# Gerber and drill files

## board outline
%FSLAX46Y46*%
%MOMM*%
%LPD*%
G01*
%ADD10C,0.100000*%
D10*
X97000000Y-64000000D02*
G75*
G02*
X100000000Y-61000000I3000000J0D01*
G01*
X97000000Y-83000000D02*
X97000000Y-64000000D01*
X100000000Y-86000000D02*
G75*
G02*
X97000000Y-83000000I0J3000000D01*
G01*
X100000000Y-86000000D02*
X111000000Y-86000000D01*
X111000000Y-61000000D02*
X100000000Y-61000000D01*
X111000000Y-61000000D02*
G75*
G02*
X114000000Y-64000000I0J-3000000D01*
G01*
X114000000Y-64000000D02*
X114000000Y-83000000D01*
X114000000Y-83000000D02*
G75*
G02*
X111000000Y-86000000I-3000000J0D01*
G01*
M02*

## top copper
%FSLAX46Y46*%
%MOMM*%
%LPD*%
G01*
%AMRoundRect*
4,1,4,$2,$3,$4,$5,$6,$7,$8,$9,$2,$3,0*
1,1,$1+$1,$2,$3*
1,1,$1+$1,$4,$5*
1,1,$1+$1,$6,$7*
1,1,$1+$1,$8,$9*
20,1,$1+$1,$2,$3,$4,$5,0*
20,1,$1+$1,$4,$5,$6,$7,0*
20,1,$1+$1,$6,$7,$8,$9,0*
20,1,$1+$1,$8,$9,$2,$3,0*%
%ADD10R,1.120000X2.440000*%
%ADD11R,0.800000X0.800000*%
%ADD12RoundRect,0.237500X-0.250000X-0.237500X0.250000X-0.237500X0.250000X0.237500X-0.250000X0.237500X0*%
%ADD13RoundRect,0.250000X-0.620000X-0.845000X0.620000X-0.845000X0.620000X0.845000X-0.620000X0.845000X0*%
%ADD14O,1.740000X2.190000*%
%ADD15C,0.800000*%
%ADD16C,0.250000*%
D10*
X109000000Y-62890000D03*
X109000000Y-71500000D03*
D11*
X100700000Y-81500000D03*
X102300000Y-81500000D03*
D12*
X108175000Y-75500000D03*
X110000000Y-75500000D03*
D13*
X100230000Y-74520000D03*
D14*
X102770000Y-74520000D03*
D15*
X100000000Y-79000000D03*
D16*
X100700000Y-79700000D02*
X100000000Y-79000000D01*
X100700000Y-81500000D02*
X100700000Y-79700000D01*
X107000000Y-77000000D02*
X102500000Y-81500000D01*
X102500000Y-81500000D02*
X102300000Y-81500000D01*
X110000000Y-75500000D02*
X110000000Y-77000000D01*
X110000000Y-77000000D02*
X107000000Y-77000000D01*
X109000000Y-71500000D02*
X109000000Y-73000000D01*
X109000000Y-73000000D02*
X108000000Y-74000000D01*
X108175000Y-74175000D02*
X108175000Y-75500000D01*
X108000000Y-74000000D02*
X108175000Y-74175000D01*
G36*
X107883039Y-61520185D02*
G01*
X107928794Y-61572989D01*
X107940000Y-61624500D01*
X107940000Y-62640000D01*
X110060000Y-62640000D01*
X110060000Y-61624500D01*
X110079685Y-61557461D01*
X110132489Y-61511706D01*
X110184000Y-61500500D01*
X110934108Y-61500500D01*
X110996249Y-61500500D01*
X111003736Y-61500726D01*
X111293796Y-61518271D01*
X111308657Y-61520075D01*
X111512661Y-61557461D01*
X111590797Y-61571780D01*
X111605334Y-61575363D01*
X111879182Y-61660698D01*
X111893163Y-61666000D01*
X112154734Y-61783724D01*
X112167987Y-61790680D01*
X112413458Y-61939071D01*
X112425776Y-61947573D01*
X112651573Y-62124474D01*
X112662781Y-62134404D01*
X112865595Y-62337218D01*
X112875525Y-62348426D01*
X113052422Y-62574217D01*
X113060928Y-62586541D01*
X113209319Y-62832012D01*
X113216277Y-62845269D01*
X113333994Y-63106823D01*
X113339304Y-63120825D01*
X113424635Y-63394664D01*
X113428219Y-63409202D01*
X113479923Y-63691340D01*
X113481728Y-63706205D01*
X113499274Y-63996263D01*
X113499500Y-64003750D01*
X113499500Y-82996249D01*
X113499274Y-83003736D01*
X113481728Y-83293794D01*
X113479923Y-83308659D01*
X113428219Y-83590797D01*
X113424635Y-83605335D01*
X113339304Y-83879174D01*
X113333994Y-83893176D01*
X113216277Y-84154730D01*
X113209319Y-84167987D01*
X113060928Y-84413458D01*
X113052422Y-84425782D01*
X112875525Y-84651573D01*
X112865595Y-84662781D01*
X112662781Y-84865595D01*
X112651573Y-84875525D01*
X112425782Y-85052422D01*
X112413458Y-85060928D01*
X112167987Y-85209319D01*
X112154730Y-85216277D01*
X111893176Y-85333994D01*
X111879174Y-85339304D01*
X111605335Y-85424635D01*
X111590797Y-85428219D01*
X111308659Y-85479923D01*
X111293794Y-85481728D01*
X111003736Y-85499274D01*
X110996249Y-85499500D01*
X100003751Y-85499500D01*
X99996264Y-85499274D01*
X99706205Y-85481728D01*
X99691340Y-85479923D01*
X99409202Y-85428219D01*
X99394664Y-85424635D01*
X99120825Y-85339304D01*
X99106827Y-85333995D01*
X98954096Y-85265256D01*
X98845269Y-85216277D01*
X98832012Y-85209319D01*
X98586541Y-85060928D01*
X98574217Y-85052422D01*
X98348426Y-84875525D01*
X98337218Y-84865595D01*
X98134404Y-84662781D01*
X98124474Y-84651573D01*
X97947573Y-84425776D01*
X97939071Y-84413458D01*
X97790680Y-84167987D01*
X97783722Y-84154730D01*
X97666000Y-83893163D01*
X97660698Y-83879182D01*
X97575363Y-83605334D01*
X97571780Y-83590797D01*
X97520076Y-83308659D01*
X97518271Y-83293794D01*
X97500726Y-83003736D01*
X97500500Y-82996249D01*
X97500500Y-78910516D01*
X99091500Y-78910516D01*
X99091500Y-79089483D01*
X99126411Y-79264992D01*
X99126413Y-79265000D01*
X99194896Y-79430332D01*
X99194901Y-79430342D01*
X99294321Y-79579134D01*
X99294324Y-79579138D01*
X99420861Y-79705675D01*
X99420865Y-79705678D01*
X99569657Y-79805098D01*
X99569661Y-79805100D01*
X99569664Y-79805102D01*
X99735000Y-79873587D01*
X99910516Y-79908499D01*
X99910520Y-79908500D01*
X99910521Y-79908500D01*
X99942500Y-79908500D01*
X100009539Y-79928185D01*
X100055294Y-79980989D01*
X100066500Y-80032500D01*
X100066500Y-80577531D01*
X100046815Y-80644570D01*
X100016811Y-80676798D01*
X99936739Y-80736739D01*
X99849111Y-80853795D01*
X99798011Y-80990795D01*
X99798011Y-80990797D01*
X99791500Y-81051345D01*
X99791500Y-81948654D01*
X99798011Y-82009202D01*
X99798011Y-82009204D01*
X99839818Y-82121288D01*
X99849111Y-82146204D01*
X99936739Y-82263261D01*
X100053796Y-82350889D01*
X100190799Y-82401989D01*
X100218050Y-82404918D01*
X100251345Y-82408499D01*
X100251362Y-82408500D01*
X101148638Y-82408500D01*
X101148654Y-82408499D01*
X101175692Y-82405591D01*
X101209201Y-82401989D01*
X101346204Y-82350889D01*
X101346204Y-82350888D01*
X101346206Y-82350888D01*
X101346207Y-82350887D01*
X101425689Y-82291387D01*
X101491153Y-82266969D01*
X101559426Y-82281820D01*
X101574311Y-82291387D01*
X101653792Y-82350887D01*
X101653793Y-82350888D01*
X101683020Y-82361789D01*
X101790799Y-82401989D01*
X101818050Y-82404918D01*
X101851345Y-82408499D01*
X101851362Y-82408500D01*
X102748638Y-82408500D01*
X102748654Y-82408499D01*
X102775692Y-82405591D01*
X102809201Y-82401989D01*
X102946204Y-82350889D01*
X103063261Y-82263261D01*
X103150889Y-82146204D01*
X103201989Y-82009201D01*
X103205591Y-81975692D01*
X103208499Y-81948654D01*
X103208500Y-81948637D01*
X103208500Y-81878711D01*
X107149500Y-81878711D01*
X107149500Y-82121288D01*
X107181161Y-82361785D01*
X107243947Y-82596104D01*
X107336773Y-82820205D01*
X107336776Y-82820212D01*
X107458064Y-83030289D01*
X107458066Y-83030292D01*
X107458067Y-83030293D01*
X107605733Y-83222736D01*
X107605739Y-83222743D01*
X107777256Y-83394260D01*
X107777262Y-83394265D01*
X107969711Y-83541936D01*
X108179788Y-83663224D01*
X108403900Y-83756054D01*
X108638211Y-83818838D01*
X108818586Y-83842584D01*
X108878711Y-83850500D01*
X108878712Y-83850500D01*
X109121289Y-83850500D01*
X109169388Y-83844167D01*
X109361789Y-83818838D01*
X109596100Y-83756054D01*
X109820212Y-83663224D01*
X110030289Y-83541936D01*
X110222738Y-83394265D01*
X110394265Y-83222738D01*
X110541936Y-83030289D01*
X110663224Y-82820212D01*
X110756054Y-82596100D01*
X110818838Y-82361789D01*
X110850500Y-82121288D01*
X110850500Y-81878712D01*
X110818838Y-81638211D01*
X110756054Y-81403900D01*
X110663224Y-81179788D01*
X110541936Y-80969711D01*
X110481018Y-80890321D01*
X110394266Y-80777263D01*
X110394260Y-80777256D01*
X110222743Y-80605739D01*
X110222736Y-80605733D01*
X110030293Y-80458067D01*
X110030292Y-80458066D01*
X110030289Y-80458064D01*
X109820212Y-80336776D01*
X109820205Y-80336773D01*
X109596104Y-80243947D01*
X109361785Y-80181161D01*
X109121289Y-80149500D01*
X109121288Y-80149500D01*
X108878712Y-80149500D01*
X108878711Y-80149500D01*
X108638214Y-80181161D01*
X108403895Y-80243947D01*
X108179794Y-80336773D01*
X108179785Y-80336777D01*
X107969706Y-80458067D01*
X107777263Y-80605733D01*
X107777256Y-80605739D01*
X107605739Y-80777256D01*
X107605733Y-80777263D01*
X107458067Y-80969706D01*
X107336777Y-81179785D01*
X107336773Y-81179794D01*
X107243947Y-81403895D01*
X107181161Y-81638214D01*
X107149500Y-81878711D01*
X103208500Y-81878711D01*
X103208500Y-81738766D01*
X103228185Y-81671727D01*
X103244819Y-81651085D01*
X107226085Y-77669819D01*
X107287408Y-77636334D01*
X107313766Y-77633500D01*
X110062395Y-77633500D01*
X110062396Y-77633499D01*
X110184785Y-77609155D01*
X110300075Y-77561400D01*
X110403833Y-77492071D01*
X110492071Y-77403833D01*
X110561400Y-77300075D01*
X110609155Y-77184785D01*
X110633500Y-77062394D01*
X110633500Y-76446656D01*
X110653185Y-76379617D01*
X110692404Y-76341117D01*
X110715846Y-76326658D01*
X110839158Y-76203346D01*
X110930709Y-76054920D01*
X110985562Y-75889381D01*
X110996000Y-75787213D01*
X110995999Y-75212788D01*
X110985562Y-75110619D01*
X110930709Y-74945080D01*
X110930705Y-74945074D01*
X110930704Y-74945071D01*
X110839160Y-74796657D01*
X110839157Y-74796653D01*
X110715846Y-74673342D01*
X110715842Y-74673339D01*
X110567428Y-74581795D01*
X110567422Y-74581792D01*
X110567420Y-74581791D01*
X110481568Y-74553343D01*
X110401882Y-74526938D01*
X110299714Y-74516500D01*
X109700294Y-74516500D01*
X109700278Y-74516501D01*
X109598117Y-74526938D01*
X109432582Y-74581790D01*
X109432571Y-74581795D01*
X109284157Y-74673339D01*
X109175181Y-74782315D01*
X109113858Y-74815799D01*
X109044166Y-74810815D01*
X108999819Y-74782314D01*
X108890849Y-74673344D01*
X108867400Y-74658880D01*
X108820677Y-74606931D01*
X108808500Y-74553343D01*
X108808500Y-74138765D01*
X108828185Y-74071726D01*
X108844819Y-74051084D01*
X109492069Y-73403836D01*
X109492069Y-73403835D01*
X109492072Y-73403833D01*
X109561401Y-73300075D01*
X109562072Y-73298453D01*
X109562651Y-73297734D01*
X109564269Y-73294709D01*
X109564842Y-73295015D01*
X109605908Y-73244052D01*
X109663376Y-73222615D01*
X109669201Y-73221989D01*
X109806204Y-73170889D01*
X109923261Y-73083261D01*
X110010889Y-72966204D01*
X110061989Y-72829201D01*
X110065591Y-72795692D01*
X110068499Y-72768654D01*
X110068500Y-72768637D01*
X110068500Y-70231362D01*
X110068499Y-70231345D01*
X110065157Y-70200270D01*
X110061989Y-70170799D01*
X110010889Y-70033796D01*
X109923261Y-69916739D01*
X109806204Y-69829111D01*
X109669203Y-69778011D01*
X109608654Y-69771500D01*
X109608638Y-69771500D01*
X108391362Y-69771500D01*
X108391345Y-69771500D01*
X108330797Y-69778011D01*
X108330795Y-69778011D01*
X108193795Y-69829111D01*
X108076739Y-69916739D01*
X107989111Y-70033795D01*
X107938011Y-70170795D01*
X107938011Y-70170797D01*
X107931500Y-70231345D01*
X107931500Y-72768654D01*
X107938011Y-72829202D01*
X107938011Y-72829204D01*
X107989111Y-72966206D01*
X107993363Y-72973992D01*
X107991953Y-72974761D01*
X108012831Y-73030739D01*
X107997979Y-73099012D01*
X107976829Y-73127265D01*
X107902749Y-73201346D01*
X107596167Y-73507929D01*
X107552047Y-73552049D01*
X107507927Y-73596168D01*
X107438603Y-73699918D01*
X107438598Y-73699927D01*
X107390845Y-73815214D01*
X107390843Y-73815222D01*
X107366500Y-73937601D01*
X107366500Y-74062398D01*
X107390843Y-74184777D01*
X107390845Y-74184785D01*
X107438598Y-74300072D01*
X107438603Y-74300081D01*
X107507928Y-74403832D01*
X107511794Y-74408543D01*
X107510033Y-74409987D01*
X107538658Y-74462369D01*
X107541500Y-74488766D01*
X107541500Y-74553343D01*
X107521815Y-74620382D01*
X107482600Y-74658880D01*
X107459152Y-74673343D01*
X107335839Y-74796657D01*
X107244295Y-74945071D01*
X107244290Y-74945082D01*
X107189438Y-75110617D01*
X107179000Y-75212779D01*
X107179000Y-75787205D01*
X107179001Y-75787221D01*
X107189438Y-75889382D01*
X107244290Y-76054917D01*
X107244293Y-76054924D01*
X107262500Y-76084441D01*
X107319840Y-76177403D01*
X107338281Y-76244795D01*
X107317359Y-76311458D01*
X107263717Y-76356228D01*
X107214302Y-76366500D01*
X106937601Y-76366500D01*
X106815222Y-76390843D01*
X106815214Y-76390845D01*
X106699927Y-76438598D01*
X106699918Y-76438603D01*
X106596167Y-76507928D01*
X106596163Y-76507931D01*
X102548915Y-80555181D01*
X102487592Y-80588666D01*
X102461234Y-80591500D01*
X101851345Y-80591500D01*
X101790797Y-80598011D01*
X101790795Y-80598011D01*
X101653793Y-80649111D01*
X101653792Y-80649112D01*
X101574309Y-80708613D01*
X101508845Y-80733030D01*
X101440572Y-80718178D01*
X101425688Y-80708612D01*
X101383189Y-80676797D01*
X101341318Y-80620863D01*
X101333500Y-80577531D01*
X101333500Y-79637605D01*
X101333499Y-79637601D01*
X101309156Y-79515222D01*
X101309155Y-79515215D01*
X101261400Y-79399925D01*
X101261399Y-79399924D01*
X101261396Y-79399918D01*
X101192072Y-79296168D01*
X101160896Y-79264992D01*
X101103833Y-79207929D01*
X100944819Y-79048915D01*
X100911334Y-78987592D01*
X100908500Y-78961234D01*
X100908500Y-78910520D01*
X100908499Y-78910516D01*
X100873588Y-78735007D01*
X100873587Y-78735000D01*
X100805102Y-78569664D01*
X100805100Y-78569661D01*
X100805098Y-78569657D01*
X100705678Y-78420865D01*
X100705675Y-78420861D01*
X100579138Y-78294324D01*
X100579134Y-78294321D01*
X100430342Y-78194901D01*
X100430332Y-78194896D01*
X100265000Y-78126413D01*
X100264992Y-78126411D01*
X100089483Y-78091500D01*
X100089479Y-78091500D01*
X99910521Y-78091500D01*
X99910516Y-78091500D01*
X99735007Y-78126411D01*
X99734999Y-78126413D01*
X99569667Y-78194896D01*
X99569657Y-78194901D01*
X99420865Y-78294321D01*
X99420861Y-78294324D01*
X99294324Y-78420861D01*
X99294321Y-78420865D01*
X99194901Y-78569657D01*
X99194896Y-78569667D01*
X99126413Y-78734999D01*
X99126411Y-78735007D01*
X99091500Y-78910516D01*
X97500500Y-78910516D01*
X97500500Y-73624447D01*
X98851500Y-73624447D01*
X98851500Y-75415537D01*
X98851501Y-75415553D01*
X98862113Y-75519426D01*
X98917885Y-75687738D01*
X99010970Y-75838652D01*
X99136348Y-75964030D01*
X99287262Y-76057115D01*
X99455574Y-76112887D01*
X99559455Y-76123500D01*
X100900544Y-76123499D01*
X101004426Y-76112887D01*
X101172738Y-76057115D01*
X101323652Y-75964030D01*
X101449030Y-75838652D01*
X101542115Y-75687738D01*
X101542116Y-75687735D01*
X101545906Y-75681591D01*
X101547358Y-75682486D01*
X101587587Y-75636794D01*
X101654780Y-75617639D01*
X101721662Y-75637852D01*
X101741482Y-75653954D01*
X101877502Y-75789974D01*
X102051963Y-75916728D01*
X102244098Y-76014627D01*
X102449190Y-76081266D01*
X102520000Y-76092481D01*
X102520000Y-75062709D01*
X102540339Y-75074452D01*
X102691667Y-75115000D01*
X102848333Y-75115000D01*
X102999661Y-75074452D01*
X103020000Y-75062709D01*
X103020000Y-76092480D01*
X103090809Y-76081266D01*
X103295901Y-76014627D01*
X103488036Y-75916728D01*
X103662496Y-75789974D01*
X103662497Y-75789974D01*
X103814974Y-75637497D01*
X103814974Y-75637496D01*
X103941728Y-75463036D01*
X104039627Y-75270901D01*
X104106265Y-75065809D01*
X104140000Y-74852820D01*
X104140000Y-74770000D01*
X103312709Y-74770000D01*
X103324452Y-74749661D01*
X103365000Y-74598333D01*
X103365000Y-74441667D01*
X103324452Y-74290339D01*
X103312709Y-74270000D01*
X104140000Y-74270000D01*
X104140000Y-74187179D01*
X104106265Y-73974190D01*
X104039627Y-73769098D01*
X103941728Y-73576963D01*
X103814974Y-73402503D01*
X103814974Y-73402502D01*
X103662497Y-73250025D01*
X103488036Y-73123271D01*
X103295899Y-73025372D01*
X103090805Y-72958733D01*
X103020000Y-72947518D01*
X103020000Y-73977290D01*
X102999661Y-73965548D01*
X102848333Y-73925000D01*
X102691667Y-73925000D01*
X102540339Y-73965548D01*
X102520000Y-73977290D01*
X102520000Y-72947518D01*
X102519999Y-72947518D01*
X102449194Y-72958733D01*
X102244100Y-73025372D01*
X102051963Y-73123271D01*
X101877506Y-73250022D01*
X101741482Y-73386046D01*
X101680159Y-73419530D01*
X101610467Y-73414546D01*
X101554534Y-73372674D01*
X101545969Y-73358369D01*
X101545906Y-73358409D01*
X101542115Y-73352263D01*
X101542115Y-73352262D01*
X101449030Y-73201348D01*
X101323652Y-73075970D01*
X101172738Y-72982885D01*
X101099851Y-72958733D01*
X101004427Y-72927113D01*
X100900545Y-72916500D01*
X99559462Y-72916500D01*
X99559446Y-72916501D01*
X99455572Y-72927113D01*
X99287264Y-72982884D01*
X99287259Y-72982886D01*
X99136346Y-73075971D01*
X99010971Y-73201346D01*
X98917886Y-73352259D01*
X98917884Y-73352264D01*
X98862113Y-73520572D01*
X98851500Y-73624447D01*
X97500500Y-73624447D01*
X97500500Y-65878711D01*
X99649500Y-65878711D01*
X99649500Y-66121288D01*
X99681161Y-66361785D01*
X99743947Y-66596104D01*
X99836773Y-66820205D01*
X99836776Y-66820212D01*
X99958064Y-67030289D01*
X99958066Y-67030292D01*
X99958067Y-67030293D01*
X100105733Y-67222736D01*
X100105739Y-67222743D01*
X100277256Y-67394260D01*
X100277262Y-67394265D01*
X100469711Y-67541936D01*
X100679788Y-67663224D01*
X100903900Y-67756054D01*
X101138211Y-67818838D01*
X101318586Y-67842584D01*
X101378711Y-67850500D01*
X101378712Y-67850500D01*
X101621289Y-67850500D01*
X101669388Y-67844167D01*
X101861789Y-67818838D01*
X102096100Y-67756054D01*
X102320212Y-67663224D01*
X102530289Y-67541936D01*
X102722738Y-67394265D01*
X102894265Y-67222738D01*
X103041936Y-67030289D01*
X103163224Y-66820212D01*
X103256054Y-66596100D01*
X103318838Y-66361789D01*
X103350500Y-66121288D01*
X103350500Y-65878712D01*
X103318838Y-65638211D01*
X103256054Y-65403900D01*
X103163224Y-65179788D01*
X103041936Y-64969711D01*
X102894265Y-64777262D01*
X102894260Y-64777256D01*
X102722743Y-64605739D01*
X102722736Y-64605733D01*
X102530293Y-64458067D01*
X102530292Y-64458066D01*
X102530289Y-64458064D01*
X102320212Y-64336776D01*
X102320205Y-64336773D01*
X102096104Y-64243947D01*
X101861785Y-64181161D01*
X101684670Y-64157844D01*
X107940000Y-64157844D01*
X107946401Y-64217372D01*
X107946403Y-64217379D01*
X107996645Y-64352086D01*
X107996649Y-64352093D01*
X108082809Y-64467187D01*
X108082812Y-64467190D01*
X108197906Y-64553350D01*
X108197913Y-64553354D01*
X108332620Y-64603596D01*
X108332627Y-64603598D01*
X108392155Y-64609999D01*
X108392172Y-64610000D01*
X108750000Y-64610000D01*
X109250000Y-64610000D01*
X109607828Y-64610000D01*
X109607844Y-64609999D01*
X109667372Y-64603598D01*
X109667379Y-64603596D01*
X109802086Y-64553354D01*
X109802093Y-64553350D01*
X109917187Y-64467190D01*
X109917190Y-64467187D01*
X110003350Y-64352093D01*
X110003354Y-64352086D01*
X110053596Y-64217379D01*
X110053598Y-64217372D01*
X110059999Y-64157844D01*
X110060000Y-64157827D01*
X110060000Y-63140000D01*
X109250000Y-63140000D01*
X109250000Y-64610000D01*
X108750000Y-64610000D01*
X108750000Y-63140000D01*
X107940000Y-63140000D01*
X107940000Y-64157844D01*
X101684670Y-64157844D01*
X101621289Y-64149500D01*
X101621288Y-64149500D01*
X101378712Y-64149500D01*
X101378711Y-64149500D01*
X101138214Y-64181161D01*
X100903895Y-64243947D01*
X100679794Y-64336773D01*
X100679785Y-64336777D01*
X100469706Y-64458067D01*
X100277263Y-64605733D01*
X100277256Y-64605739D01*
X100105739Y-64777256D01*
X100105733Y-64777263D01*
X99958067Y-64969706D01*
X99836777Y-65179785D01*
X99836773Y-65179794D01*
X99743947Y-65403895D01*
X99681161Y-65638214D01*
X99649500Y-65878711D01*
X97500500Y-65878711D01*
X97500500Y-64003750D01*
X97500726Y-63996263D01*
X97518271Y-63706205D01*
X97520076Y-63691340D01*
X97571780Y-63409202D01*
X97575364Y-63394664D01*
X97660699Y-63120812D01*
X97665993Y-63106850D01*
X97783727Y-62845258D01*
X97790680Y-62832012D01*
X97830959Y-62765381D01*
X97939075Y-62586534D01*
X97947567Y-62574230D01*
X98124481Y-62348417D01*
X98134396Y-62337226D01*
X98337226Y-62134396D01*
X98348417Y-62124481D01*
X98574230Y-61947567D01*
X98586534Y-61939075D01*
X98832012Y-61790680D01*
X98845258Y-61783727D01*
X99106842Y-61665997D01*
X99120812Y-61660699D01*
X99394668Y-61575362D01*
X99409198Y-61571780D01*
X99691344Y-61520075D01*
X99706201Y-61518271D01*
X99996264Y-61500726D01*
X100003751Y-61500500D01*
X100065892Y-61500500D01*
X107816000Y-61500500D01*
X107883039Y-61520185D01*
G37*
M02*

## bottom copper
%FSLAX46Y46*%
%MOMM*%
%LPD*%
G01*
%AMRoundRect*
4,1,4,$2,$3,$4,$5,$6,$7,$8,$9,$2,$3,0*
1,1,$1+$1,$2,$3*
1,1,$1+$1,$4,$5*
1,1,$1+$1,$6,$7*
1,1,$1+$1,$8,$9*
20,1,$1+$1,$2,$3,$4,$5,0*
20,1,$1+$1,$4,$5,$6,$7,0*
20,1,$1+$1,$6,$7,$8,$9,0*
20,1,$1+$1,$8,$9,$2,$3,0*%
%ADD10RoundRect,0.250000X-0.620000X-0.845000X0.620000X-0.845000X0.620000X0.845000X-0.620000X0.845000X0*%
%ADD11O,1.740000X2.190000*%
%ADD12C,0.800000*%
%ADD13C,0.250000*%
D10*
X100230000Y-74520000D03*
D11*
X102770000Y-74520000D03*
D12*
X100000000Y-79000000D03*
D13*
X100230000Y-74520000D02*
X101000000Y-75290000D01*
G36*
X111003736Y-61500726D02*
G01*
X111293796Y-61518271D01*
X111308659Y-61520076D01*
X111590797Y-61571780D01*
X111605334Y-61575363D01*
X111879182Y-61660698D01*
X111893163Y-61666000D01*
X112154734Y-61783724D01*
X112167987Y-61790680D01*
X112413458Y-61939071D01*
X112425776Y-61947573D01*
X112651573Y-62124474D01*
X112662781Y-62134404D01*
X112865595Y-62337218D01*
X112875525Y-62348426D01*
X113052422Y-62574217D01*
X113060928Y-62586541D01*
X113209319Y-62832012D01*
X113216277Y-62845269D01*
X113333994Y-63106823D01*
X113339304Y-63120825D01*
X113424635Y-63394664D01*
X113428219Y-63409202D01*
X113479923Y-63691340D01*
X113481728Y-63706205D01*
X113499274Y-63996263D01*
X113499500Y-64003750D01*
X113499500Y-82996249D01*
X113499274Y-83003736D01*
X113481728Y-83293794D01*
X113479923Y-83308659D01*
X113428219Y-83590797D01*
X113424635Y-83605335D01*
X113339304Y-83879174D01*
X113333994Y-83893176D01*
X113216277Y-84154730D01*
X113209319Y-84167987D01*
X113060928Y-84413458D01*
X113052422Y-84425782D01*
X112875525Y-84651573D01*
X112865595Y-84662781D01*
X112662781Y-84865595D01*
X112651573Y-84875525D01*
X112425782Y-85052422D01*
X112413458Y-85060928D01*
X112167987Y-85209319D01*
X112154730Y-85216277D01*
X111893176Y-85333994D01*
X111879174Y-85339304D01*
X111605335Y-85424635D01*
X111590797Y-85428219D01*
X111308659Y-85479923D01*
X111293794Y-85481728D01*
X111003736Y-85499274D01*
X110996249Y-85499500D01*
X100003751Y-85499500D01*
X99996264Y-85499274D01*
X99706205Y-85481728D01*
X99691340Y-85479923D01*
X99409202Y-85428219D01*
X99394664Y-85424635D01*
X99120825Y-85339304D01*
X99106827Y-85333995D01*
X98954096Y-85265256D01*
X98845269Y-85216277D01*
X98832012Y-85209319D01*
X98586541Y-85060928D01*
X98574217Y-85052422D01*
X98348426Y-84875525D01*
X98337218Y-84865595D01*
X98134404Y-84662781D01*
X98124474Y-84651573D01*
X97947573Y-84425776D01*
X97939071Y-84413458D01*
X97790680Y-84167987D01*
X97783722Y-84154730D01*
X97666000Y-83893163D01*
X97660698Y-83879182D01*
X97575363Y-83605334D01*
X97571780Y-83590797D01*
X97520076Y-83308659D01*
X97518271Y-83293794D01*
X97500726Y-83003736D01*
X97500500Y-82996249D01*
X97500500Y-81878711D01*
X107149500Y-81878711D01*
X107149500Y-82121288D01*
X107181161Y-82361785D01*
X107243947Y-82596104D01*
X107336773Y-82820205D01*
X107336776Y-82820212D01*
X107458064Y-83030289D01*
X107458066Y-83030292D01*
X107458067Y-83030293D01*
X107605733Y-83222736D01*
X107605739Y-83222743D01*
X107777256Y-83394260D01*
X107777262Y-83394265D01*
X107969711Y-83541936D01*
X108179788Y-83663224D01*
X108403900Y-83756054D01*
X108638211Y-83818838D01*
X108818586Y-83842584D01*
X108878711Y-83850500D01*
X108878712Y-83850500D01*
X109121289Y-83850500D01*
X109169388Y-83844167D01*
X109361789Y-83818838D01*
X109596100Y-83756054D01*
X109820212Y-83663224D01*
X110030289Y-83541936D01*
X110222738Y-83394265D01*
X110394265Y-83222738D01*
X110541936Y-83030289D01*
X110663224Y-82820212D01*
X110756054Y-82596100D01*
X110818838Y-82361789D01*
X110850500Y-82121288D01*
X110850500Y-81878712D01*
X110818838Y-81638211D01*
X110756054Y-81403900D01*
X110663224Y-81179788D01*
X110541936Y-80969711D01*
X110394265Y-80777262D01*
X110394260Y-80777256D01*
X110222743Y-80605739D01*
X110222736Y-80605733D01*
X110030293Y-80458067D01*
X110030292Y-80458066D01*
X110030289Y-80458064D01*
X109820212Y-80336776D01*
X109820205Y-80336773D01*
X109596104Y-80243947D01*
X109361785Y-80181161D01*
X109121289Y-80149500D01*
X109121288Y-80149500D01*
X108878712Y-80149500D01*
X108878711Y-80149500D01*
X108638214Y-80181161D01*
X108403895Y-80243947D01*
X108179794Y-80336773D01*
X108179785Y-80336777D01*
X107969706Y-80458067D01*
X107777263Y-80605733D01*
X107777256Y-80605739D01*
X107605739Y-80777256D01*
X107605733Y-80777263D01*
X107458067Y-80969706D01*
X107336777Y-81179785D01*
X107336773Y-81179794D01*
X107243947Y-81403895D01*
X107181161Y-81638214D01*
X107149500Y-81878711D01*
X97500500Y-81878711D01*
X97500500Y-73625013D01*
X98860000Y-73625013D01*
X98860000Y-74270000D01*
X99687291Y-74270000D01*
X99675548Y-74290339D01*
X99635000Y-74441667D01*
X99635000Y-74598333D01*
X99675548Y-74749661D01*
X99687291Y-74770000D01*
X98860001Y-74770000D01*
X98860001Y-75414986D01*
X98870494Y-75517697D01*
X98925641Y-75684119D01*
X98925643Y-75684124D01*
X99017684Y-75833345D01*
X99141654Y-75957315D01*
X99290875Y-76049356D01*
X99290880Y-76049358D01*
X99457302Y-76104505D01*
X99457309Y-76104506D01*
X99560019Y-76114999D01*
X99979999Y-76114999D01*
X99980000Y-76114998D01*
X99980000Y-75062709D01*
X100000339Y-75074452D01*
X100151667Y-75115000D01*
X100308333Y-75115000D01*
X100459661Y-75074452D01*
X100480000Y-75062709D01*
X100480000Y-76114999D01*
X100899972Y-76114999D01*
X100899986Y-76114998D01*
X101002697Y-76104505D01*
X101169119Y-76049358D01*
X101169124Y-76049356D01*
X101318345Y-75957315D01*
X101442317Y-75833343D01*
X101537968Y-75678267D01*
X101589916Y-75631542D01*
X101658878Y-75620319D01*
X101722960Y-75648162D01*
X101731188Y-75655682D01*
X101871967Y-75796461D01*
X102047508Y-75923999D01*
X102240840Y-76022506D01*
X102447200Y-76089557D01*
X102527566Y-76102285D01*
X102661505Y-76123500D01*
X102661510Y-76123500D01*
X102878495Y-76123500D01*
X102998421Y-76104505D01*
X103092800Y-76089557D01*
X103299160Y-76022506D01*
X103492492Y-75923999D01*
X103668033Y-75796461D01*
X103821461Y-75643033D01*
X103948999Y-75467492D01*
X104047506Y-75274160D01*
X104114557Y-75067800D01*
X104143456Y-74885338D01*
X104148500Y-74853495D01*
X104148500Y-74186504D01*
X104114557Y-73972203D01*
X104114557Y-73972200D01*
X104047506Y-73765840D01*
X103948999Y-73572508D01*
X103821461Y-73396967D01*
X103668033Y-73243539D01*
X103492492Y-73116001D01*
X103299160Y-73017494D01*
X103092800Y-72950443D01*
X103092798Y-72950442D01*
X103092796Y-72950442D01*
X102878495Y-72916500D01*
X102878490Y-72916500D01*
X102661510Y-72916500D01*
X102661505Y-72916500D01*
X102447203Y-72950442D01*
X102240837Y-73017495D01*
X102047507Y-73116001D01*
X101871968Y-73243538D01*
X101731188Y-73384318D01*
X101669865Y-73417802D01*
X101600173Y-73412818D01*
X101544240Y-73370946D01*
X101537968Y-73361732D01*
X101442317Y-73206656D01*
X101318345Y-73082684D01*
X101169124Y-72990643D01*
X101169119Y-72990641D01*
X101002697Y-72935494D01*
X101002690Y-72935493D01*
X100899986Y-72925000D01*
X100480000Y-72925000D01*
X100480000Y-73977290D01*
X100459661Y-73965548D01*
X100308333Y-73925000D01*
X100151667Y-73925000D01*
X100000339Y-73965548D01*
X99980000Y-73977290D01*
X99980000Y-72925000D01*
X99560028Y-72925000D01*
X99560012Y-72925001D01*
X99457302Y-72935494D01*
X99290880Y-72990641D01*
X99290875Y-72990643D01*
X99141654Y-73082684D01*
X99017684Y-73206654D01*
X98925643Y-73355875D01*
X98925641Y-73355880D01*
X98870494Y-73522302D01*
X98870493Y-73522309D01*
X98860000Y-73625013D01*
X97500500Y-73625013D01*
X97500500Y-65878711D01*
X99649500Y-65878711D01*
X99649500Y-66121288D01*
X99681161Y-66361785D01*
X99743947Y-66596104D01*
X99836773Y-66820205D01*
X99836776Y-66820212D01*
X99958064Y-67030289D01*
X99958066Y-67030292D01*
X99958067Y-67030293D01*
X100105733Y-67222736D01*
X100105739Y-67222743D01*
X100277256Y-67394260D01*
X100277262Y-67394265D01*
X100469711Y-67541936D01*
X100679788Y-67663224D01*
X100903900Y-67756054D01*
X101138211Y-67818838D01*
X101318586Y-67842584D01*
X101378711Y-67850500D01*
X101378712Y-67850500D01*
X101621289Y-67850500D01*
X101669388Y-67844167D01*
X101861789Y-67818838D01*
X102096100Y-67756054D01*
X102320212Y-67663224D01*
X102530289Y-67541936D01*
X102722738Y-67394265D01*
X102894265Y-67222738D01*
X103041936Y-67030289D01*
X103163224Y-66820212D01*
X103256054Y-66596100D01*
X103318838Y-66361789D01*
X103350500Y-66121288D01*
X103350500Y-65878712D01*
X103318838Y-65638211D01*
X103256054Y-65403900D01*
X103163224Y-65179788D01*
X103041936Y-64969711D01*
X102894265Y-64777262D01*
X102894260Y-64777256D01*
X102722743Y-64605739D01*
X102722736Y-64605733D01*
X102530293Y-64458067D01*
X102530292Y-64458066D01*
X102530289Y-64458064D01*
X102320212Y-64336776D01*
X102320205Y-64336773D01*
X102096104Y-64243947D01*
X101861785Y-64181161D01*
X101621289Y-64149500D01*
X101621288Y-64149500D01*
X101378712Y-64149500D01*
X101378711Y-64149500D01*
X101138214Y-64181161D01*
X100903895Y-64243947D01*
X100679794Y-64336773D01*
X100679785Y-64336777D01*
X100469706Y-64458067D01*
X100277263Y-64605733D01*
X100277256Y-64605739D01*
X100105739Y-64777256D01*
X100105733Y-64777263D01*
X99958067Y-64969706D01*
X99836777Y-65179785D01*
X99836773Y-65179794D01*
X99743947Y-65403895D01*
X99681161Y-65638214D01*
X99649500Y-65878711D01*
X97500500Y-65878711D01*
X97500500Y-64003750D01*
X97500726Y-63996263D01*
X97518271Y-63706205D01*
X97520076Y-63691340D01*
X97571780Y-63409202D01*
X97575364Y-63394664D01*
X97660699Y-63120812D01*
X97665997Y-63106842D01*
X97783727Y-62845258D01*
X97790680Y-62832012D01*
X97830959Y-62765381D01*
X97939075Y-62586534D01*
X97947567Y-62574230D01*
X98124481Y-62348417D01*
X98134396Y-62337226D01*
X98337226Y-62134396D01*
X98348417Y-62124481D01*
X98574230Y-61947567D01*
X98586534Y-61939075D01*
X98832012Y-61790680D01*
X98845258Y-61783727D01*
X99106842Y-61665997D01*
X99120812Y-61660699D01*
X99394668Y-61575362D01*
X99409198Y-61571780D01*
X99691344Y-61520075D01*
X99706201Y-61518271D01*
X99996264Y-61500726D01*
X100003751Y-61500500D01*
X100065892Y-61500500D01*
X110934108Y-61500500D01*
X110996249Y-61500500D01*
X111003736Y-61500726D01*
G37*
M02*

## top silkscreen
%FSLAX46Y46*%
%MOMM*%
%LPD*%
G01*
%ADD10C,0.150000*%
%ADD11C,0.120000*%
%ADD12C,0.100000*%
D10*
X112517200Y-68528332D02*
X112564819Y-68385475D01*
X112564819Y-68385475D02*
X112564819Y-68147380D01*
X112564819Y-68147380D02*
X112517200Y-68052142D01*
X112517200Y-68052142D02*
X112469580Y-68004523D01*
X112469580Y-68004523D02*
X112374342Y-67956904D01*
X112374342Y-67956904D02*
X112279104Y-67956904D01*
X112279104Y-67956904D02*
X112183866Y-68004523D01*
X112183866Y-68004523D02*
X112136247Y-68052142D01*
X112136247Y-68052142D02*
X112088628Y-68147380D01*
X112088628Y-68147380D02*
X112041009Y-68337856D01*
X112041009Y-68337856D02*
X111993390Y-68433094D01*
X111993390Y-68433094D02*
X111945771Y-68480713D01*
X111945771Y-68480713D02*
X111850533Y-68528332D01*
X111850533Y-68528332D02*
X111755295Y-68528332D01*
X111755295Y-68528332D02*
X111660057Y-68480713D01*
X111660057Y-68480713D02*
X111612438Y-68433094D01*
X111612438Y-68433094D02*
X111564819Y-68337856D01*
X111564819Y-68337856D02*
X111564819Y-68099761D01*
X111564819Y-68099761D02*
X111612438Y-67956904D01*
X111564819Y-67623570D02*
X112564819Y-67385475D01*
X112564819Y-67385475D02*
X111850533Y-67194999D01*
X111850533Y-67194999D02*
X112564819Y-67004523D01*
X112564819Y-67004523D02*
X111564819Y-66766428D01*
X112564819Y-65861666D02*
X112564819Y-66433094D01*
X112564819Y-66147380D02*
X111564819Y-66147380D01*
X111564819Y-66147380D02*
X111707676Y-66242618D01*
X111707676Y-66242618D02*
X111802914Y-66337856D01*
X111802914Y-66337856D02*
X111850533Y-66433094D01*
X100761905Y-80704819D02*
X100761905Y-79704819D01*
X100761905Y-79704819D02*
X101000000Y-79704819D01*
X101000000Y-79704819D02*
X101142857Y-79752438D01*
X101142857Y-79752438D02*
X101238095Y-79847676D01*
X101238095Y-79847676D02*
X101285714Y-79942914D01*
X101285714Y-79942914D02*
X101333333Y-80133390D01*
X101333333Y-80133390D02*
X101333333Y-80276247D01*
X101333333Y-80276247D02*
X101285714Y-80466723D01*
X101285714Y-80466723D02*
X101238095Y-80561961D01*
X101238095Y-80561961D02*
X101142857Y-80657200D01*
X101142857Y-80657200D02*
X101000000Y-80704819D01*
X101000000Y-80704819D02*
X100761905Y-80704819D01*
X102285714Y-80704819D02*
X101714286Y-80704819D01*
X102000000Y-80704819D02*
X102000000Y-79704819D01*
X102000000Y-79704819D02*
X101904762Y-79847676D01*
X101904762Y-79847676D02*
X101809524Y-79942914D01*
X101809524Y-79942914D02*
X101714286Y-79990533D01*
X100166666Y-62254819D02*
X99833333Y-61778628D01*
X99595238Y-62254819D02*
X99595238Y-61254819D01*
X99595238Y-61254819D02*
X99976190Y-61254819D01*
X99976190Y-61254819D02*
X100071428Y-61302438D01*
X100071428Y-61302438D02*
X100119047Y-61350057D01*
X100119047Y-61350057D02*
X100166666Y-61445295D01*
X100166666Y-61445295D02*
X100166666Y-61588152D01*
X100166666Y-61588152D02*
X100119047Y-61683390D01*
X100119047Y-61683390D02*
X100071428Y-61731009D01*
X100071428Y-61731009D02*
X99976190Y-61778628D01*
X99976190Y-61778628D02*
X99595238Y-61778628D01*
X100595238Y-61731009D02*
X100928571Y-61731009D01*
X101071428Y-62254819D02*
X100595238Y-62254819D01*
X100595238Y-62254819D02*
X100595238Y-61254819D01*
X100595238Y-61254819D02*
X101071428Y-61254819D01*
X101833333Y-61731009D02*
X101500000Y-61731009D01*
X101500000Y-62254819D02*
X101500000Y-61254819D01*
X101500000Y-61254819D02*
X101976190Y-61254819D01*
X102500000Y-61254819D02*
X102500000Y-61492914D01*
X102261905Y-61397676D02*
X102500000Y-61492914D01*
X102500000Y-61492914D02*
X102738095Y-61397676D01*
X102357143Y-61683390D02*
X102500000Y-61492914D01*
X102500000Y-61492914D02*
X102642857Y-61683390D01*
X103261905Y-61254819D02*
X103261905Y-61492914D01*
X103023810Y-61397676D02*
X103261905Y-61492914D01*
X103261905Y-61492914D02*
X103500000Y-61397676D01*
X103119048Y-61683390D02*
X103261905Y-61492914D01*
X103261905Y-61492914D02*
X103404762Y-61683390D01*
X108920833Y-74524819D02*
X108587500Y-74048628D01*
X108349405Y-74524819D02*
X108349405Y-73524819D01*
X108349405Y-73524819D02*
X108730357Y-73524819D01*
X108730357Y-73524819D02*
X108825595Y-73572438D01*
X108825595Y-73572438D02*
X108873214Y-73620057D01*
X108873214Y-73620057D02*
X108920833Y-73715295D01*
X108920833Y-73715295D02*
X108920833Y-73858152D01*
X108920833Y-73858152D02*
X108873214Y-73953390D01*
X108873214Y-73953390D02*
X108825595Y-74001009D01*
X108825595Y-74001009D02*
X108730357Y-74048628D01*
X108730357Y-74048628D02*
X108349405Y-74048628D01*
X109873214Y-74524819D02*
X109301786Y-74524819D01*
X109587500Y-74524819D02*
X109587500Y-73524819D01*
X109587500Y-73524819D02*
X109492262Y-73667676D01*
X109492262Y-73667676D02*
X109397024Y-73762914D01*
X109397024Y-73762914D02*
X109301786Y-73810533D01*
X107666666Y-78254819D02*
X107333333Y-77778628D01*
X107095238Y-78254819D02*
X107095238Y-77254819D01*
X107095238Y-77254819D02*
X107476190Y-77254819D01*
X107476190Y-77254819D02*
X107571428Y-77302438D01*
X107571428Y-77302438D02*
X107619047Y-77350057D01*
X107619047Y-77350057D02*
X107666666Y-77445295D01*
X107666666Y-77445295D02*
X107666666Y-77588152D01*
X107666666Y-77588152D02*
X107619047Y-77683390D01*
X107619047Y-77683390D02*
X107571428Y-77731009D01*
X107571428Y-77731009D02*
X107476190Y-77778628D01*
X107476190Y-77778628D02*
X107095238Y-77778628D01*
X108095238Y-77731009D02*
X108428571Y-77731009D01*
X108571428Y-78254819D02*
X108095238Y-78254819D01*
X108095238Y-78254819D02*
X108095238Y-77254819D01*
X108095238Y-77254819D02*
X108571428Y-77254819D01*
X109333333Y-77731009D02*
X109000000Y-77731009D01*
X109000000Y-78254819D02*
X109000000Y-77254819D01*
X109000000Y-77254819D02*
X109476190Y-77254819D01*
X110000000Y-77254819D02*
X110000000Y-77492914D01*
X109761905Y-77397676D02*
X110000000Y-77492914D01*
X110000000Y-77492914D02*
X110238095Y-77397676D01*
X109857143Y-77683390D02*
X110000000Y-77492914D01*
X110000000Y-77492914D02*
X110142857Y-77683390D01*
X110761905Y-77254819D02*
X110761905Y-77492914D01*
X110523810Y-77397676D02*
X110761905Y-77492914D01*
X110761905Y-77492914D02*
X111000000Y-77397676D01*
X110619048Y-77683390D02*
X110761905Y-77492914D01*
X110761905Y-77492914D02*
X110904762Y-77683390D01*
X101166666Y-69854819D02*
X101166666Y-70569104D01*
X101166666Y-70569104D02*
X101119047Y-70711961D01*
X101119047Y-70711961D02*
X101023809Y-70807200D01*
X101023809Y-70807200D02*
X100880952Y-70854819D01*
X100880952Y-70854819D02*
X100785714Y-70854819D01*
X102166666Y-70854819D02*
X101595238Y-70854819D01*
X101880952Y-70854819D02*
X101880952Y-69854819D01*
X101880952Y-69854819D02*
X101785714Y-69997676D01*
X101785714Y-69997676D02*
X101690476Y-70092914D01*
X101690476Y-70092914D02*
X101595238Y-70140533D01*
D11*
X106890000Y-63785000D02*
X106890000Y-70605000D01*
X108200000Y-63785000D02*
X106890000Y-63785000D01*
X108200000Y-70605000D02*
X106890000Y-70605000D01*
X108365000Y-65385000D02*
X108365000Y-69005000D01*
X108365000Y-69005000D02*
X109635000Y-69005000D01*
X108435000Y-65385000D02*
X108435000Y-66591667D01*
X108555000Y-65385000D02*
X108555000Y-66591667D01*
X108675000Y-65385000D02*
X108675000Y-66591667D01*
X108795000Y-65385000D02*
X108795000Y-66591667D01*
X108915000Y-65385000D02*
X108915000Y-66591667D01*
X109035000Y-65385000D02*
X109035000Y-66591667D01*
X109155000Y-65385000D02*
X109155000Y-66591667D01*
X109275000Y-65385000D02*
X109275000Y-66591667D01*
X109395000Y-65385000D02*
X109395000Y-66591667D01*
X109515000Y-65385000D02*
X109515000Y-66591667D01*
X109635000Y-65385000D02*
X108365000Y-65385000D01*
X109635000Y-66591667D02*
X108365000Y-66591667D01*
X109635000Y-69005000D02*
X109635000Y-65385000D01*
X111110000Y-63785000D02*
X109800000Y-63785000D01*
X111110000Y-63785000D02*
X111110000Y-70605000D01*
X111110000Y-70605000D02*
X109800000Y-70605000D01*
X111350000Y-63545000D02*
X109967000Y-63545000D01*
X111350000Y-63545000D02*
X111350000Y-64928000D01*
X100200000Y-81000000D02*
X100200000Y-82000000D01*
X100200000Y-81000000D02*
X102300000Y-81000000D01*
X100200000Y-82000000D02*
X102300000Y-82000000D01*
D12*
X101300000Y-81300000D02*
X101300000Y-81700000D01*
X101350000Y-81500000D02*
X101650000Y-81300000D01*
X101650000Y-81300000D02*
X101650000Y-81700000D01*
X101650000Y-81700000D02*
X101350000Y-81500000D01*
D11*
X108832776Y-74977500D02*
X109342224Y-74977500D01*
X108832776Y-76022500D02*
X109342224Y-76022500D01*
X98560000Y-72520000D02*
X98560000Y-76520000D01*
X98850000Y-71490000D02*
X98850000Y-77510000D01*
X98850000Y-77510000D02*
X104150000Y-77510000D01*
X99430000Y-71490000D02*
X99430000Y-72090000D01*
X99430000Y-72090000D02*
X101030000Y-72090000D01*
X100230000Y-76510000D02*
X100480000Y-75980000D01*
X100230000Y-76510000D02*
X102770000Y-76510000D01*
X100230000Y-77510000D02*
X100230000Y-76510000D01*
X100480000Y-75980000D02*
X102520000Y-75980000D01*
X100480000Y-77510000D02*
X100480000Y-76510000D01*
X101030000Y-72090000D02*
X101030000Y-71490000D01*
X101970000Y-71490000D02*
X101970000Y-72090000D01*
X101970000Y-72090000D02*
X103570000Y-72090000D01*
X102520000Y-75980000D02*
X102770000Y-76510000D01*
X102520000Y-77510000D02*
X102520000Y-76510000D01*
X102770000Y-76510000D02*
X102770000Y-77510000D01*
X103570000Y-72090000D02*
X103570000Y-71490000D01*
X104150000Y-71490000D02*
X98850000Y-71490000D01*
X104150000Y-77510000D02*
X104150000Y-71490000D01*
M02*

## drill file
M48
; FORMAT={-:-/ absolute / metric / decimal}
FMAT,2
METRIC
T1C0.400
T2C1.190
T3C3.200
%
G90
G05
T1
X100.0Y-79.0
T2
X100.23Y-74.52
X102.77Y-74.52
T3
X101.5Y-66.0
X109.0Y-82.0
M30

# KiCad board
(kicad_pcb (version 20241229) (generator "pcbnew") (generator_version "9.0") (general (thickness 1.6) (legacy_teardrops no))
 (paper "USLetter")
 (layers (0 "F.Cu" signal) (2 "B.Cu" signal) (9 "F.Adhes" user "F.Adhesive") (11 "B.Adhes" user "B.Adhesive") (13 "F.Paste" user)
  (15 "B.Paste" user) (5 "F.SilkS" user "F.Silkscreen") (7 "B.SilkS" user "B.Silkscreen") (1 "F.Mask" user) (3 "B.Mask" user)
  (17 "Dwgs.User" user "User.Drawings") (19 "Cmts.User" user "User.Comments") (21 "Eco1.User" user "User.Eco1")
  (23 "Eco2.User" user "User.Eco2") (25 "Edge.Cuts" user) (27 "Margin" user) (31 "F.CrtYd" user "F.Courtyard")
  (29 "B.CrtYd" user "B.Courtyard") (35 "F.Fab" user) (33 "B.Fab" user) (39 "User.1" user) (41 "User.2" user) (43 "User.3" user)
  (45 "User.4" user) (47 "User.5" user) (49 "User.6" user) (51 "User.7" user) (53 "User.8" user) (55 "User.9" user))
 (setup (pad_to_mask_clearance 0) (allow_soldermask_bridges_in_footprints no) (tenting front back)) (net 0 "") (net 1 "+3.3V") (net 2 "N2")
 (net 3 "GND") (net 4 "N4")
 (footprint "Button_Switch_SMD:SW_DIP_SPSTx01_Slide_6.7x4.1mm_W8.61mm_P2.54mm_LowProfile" (layer "F.Cu") (at 109 67.195 -90)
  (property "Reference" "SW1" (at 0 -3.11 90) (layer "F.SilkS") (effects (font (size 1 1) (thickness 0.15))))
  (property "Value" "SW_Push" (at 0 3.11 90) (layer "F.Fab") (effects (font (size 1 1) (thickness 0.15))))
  (fp_line (start -3.41 2.11) (end 3.41 2.11) (stroke (width 0.12) (type solid)) (layer "F.SilkS"))
  (fp_line (start -3.41 0.8) (end -3.41 2.11) (stroke (width 0.12) (type solid)) (layer "F.SilkS"))
  (fp_line (start 3.41 0.8) (end 3.41 2.11) (stroke (width 0.12) (type solid)) (layer "F.SilkS"))
  (fp_line (start -1.81 0.635) (end 1.81 0.635) (stroke (width 0.12) (type solid)) (layer "F.SilkS"))
  (fp_line (start 1.81 0.635) (end 1.81 -0.635) (stroke (width 0.12) (type solid)) (layer "F.SilkS"))
  (fp_line (start -1.81 0.565) (end -0.603333 0.565) (stroke (width 0.12) (type solid)) (layer "F.SilkS"))
  (fp_line (start -1.81 0.445) (end -0.603333 0.445) (stroke (width 0.12) (type solid)) (layer "F.SilkS"))
  (fp_line (start -1.81 0.325) (end -0.603333 0.325) (stroke (width 0.12) (type solid)) (layer "F.SilkS"))
  (fp_line (start -1.81 0.205) (end -0.603333 0.205) (stroke (width 0.12) (type solid)) (layer "F.SilkS"))
  (fp_line (start -1.81 0.085) (end -0.603333 0.085) (stroke (width 0.12) (type solid)) (layer "F.SilkS"))
  (fp_line (start -1.81 -0.035) (end -0.603333 -0.035) (stroke (width 0.12) (type solid)) (layer "F.SilkS"))
  (fp_line (start -1.81 -0.155) (end -0.603333 -0.155) (stroke (width 0.12) (type solid)) (layer "F.SilkS"))
  (fp_line (start -1.81 -0.275) (end -0.603333 -0.275) (stroke (width 0.12) (type solid)) (layer "F.SilkS"))
  (fp_line (start -1.81 -0.395) (end -0.603333 -0.395) (stroke (width 0.12) (type solid)) (layer "F.SilkS"))
  (fp_line (start -1.81 -0.515) (end -0.603333 -0.515) (stroke (width 0.12) (type solid)) (layer "F.SilkS"))
  (fp_line (start -1.81 -0.635) (end -1.81 0.635) (stroke (width 0.12) (type solid)) (layer "F.SilkS"))
  (fp_line (start -0.603333 -0.635) (end -0.603333 0.635) (stroke (width 0.12) (type solid)) (layer "F.SilkS"))
  (fp_line (start 1.81 -0.635) (end -1.81 -0.635) (stroke (width 0.12) (type solid)) (layer "F.SilkS"))
  (fp_line (start -3.41 -2.11) (end -3.41 -0.8) (stroke (width 0.12) (type solid)) (layer "F.SilkS"))
  (fp_line (start -3.41 -2.11) (end 3.41 -2.11) (stroke (width 0.12) (type solid)) (layer "F.SilkS"))
  (fp_line (start 3.41 -2.11) (end 3.41 -0.8) (stroke (width 0.12) (type solid)) (layer "F.SilkS"))
  (fp_line (start -3.65 -2.35) (end -3.65 -0.967) (stroke (width 0.12) (type solid)) (layer "F.SilkS"))
  (fp_line (start -3.65 -2.35) (end -2.267 -2.35) (stroke (width 0.12) (type solid)) (layer "F.SilkS"))
  (pad "1" smd rect (at -4.305 0 270) (size 2.44 1.12) (layers "F.Cu" "F.Mask" "F.Paste") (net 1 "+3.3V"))
  (pad "2" smd rect (at 4.305 0 270) (size 2.44 1.12) (layers "F.Cu" "F.Mask" "F.Paste") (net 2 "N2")))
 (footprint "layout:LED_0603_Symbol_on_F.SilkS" (layer "F.Cu") (at 101.5 81.5)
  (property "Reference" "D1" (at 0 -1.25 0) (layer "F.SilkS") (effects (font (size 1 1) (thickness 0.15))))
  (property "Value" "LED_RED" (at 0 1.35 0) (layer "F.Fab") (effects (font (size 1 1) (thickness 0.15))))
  (fp_line (start -1.3 -0.5) (end -1.3 0.5) (stroke (width 0.12) (type solid)) (layer "F.SilkS"))
  (fp_line (start -1.3 -0.5) (end 0.8 -0.5) (stroke (width 0.12) (type solid)) (layer "F.SilkS"))
  (fp_line (start -1.3 0.5) (end 0.8 0.5) (stroke (width 0.12) (type solid)) (layer "F.SilkS"))
  (fp_line (start -0.2 -0.2) (end -0.2 0.2) (stroke (width 0.1) (type solid)) (layer "F.SilkS"))
  (fp_line (start -0.15 0) (end 0.15 -0.2) (stroke (width 0.1) (type solid)) (layer "F.SilkS"))
  (fp_line (start 0.15 -0.2) (end 0.15 0.2) (stroke (width 0.1) (type solid)) (layer "F.SilkS"))
  (fp_line (start 0.15 0.2) (end -0.15 0) (stroke (width 0.1) (type solid)) (layer "F.SilkS"))
  (pad "1" smd rect (at -0.8 0 180) (size 0.8 0.8) (layers "F.Cu" "F.Mask" "F.Paste") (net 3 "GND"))
  (pad "2" smd rect (at 0.8 0 180) (size 0.8 0.8) (layers "F.Cu" "F.Mask" "F.Paste") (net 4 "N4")))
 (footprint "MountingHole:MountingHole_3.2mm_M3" (layer "F.Cu") (at 101.5 66)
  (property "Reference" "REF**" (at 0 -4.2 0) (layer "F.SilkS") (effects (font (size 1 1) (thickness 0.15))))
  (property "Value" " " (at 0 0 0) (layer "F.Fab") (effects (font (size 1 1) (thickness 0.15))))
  (pad "" np_thru_hole circle (at 0 0) (size 3.2 3.2) (drill 3.2) (layers "*.Cu" "*.Mask")))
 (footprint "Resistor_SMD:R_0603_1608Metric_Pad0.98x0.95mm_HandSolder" (layer "F.Cu") (at 109.0875 75.5)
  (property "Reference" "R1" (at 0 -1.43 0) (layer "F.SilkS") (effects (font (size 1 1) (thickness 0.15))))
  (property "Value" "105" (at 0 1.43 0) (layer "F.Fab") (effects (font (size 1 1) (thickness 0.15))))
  (fp_line (start -0.254724 -0.5225) (end 0.254724 -0.5225) (stroke (width 0.12) (type solid)) (layer "F.SilkS"))
  (fp_line (start -0.254724 0.5225) (end 0.254724 0.5225) (stroke (width 0.12) (type solid)) (layer "F.SilkS"))
  (pad "1" smd roundrect (at -0.9125 0) (size 0.975 0.95) (layers "F.Cu" "F.Mask" "F.Paste") (roundrect_rratio 0.25) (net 2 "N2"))
  (pad "2" smd roundrect (at 0.9125 0) (size 0.975 0.95) (layers "F.Cu" "F.Mask" "F.Paste") (roundrect_rratio 0.25) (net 4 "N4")))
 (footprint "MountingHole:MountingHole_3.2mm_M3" (layer "F.Cu") (at 109 82)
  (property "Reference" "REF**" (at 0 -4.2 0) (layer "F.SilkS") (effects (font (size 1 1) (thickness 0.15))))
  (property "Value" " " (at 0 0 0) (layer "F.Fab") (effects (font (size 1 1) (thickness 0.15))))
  (pad "" np_thru_hole circle (at 0 0) (size 3.2 3.2) (drill 3.2) (layers "*.Cu" "*.Mask")))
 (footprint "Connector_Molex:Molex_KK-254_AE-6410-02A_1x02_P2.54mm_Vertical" (layer "F.Cu") (at 100.23 74.52)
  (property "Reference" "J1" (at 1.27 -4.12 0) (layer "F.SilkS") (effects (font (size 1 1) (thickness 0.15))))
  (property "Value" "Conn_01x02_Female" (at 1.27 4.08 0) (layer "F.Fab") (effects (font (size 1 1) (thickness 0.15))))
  (fp_line (start -1.67 -2) (end -1.67 2) (stroke (width 0.12) (type solid)) (layer "F.SilkS"))
  (fp_line (start -1.38 -3.03) (end -1.38 2.99) (stroke (width 0.12) (type solid)) (layer "F.SilkS"))
  (fp_line (start -1.38 2.99) (end 3.92 2.99) (stroke (width 0.12) (type solid)) (layer "F.SilkS"))
  (fp_line (start -0.8 -3.03) (end -0.8 -2.43) (stroke (width 0.12) (type solid)) (layer "F.SilkS"))
  (fp_line (start -0.8 -2.43) (end 0.8 -2.43) (stroke (width 0.12) (type solid)) (layer "F.SilkS"))
  (fp_line (start 0 1.99) (end 0.25 1.46) (stroke (width 0.12) (type solid)) (layer "F.SilkS"))
  (fp_line (start 0 1.99) (end 2.54 1.99) (stroke (width 0.12) (type solid)) (layer "F.SilkS"))
  (fp_line (start 0 2.99) (end 0 1.99) (stroke (width 0.12) (type solid)) (layer "F.SilkS"))
  (fp_line (start 0.25 1.46) (end 2.29 1.46) (stroke (width 0.12) (type solid)) (layer "F.SilkS"))
  (fp_line (start 0.25 2.99) (end 0.25 1.99) (stroke (width 0.12) (type solid)) (layer "F.SilkS"))
  (fp_line (start 0.8 -2.43) (end 0.8 -3.03) (stroke (width 0.12) (type solid)) (layer "F.SilkS"))
  (fp_line (start 1.74 -3.03) (end 1.74 -2.43) (stroke (width 0.12) (type solid)) (layer "F.SilkS"))
  (fp_line (start 1.74 -2.43) (end 3.34 -2.43) (stroke (width 0.12) (type solid)) (layer "F.SilkS"))
  (fp_line (start 2.29 1.46) (end 2.54 1.99) (stroke (width 0.12) (type solid)) (layer "F.SilkS"))
  (fp_line (start 2.29 2.99) (end 2.29 1.99) (stroke (width 0.12) (type solid)) (layer "F.SilkS"))
  (fp_line (start 2.54 1.99) (end 2.54 2.99) (stroke (width 0.12) (type solid)) (layer "F.SilkS"))
  (fp_line (start 3.34 -2.43) (end 3.34 -3.03) (stroke (width 0.12) (type solid)) (layer "F.SilkS"))
  (fp_line (start 3.92 -3.03) (end -1.38 -3.03) (stroke (width 0.12) (type solid)) (layer "F.SilkS"))
  (fp_line (start 3.92 2.99) (end 3.92 -3.03) (stroke (width 0.12) (type solid)) (layer "F.SilkS"))
  (pad "1" thru_hole roundrect (at 0 0) (size 1.74 2.19) (drill 1.19) (layers "*.Cu" "*.Mask") (remove_unused_layers no)
   (roundrect_rratio 0.143678) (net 3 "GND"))
  (pad "2" thru_hole oval (at 2.54 0) (size 1.74 2.19) (drill 1.19) (layers "*.Cu" "*.Mask") (remove_unused_layers no) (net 1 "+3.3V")))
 (gr_arc (start 97 64) (mid 97.87868 61.87868) (end 100 61) (stroke (width 0.1) (type default)) (layer "Edge.Cuts"))
 (gr_line (start 97 83) (end 97 64) (stroke (width 0.1) (type default)) (layer "Edge.Cuts"))
 (gr_arc (start 100 86) (mid 97.87868 85.12132) (end 97 83) (stroke (width 0.1) (type default)) (layer "Edge.Cuts"))
 (gr_line (start 100 86) (end 111 86) (stroke (width 0.1) (type default)) (layer "Edge.Cuts"))
 (gr_line (start 111 61) (end 100 61) (stroke (width 0.1) (type default)) (layer "Edge.Cuts"))
 (gr_arc (start 111 61) (mid 113.12132 61.87868) (end 114 64) (stroke (width 0.1) (type default)) (layer "Edge.Cuts"))
 (gr_line (start 114 64) (end 114 83) (stroke (width 0.1) (type default)) (layer "Edge.Cuts"))
 (gr_arc (start 114 83) (mid 113.12132 85.12132) (end 111 86) (stroke (width 0.1) (type default)) (layer "Edge.Cuts"))
 (segment (start 100.7 79.7) (end 100 79) (width 0.25) (layer "F.Cu") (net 3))
 (segment (start 100.7 81.5) (end 100.7 79.7) (width 0.25) (layer "F.Cu") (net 3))
 (via (at 100 79) (size 0.8) (drill 0.4) (layers "F.Cu" "B.Cu") (free yes) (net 3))
 (segment (start 100.23 74.52) (end 101 75.29) (width 0.25) (layer "B.Cu") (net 3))
 (segment (start 107 77) (end 102.5 81.5) (width 0.25) (layer "F.Cu") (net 4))
 (segment (start 102.5 81.5) (end 102.3 81.5) (width 0.25) (layer "F.Cu") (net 4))
 (segment (start 110 75.5) (end 110 77) (width 0.25) (layer "F.Cu") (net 4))
 (segment (start 110 77) (end 107 77) (width 0.25) (layer "F.Cu") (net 4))
 (segment (start 109 71.5) (end 109 73) (width 0.25) (layer "F.Cu") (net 2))
 (segment (start 109 73) (end 108 74) (width 0.25) (layer "F.Cu") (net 2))
 (segment (start 108.175 74.175) (end 108.175 75.5) (width 0.25) (layer "F.Cu") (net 2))
 (segment (start 108 74) (end 108.175 74.175) (width 0.25) (layer "F.Cu") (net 2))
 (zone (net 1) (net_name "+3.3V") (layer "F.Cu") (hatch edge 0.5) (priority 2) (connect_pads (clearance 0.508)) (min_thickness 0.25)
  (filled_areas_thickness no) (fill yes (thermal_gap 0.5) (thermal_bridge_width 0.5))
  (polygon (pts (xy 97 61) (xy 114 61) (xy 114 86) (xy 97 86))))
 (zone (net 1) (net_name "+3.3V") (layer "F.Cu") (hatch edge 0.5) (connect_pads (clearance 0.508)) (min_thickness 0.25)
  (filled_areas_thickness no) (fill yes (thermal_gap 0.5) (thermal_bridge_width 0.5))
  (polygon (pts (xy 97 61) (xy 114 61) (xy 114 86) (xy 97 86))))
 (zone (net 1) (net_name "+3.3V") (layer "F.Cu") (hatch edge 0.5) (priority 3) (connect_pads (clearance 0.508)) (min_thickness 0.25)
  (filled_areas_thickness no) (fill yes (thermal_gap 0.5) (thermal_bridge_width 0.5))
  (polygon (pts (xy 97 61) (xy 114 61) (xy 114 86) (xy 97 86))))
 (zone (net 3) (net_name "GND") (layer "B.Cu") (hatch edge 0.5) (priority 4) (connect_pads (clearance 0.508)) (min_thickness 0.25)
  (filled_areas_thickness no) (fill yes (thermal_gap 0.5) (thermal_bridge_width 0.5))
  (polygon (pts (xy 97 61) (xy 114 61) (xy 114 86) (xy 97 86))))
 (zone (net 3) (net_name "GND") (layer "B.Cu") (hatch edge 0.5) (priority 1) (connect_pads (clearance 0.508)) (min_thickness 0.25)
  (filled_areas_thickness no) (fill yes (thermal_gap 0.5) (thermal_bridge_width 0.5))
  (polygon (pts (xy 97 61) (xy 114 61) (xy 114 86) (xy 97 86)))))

